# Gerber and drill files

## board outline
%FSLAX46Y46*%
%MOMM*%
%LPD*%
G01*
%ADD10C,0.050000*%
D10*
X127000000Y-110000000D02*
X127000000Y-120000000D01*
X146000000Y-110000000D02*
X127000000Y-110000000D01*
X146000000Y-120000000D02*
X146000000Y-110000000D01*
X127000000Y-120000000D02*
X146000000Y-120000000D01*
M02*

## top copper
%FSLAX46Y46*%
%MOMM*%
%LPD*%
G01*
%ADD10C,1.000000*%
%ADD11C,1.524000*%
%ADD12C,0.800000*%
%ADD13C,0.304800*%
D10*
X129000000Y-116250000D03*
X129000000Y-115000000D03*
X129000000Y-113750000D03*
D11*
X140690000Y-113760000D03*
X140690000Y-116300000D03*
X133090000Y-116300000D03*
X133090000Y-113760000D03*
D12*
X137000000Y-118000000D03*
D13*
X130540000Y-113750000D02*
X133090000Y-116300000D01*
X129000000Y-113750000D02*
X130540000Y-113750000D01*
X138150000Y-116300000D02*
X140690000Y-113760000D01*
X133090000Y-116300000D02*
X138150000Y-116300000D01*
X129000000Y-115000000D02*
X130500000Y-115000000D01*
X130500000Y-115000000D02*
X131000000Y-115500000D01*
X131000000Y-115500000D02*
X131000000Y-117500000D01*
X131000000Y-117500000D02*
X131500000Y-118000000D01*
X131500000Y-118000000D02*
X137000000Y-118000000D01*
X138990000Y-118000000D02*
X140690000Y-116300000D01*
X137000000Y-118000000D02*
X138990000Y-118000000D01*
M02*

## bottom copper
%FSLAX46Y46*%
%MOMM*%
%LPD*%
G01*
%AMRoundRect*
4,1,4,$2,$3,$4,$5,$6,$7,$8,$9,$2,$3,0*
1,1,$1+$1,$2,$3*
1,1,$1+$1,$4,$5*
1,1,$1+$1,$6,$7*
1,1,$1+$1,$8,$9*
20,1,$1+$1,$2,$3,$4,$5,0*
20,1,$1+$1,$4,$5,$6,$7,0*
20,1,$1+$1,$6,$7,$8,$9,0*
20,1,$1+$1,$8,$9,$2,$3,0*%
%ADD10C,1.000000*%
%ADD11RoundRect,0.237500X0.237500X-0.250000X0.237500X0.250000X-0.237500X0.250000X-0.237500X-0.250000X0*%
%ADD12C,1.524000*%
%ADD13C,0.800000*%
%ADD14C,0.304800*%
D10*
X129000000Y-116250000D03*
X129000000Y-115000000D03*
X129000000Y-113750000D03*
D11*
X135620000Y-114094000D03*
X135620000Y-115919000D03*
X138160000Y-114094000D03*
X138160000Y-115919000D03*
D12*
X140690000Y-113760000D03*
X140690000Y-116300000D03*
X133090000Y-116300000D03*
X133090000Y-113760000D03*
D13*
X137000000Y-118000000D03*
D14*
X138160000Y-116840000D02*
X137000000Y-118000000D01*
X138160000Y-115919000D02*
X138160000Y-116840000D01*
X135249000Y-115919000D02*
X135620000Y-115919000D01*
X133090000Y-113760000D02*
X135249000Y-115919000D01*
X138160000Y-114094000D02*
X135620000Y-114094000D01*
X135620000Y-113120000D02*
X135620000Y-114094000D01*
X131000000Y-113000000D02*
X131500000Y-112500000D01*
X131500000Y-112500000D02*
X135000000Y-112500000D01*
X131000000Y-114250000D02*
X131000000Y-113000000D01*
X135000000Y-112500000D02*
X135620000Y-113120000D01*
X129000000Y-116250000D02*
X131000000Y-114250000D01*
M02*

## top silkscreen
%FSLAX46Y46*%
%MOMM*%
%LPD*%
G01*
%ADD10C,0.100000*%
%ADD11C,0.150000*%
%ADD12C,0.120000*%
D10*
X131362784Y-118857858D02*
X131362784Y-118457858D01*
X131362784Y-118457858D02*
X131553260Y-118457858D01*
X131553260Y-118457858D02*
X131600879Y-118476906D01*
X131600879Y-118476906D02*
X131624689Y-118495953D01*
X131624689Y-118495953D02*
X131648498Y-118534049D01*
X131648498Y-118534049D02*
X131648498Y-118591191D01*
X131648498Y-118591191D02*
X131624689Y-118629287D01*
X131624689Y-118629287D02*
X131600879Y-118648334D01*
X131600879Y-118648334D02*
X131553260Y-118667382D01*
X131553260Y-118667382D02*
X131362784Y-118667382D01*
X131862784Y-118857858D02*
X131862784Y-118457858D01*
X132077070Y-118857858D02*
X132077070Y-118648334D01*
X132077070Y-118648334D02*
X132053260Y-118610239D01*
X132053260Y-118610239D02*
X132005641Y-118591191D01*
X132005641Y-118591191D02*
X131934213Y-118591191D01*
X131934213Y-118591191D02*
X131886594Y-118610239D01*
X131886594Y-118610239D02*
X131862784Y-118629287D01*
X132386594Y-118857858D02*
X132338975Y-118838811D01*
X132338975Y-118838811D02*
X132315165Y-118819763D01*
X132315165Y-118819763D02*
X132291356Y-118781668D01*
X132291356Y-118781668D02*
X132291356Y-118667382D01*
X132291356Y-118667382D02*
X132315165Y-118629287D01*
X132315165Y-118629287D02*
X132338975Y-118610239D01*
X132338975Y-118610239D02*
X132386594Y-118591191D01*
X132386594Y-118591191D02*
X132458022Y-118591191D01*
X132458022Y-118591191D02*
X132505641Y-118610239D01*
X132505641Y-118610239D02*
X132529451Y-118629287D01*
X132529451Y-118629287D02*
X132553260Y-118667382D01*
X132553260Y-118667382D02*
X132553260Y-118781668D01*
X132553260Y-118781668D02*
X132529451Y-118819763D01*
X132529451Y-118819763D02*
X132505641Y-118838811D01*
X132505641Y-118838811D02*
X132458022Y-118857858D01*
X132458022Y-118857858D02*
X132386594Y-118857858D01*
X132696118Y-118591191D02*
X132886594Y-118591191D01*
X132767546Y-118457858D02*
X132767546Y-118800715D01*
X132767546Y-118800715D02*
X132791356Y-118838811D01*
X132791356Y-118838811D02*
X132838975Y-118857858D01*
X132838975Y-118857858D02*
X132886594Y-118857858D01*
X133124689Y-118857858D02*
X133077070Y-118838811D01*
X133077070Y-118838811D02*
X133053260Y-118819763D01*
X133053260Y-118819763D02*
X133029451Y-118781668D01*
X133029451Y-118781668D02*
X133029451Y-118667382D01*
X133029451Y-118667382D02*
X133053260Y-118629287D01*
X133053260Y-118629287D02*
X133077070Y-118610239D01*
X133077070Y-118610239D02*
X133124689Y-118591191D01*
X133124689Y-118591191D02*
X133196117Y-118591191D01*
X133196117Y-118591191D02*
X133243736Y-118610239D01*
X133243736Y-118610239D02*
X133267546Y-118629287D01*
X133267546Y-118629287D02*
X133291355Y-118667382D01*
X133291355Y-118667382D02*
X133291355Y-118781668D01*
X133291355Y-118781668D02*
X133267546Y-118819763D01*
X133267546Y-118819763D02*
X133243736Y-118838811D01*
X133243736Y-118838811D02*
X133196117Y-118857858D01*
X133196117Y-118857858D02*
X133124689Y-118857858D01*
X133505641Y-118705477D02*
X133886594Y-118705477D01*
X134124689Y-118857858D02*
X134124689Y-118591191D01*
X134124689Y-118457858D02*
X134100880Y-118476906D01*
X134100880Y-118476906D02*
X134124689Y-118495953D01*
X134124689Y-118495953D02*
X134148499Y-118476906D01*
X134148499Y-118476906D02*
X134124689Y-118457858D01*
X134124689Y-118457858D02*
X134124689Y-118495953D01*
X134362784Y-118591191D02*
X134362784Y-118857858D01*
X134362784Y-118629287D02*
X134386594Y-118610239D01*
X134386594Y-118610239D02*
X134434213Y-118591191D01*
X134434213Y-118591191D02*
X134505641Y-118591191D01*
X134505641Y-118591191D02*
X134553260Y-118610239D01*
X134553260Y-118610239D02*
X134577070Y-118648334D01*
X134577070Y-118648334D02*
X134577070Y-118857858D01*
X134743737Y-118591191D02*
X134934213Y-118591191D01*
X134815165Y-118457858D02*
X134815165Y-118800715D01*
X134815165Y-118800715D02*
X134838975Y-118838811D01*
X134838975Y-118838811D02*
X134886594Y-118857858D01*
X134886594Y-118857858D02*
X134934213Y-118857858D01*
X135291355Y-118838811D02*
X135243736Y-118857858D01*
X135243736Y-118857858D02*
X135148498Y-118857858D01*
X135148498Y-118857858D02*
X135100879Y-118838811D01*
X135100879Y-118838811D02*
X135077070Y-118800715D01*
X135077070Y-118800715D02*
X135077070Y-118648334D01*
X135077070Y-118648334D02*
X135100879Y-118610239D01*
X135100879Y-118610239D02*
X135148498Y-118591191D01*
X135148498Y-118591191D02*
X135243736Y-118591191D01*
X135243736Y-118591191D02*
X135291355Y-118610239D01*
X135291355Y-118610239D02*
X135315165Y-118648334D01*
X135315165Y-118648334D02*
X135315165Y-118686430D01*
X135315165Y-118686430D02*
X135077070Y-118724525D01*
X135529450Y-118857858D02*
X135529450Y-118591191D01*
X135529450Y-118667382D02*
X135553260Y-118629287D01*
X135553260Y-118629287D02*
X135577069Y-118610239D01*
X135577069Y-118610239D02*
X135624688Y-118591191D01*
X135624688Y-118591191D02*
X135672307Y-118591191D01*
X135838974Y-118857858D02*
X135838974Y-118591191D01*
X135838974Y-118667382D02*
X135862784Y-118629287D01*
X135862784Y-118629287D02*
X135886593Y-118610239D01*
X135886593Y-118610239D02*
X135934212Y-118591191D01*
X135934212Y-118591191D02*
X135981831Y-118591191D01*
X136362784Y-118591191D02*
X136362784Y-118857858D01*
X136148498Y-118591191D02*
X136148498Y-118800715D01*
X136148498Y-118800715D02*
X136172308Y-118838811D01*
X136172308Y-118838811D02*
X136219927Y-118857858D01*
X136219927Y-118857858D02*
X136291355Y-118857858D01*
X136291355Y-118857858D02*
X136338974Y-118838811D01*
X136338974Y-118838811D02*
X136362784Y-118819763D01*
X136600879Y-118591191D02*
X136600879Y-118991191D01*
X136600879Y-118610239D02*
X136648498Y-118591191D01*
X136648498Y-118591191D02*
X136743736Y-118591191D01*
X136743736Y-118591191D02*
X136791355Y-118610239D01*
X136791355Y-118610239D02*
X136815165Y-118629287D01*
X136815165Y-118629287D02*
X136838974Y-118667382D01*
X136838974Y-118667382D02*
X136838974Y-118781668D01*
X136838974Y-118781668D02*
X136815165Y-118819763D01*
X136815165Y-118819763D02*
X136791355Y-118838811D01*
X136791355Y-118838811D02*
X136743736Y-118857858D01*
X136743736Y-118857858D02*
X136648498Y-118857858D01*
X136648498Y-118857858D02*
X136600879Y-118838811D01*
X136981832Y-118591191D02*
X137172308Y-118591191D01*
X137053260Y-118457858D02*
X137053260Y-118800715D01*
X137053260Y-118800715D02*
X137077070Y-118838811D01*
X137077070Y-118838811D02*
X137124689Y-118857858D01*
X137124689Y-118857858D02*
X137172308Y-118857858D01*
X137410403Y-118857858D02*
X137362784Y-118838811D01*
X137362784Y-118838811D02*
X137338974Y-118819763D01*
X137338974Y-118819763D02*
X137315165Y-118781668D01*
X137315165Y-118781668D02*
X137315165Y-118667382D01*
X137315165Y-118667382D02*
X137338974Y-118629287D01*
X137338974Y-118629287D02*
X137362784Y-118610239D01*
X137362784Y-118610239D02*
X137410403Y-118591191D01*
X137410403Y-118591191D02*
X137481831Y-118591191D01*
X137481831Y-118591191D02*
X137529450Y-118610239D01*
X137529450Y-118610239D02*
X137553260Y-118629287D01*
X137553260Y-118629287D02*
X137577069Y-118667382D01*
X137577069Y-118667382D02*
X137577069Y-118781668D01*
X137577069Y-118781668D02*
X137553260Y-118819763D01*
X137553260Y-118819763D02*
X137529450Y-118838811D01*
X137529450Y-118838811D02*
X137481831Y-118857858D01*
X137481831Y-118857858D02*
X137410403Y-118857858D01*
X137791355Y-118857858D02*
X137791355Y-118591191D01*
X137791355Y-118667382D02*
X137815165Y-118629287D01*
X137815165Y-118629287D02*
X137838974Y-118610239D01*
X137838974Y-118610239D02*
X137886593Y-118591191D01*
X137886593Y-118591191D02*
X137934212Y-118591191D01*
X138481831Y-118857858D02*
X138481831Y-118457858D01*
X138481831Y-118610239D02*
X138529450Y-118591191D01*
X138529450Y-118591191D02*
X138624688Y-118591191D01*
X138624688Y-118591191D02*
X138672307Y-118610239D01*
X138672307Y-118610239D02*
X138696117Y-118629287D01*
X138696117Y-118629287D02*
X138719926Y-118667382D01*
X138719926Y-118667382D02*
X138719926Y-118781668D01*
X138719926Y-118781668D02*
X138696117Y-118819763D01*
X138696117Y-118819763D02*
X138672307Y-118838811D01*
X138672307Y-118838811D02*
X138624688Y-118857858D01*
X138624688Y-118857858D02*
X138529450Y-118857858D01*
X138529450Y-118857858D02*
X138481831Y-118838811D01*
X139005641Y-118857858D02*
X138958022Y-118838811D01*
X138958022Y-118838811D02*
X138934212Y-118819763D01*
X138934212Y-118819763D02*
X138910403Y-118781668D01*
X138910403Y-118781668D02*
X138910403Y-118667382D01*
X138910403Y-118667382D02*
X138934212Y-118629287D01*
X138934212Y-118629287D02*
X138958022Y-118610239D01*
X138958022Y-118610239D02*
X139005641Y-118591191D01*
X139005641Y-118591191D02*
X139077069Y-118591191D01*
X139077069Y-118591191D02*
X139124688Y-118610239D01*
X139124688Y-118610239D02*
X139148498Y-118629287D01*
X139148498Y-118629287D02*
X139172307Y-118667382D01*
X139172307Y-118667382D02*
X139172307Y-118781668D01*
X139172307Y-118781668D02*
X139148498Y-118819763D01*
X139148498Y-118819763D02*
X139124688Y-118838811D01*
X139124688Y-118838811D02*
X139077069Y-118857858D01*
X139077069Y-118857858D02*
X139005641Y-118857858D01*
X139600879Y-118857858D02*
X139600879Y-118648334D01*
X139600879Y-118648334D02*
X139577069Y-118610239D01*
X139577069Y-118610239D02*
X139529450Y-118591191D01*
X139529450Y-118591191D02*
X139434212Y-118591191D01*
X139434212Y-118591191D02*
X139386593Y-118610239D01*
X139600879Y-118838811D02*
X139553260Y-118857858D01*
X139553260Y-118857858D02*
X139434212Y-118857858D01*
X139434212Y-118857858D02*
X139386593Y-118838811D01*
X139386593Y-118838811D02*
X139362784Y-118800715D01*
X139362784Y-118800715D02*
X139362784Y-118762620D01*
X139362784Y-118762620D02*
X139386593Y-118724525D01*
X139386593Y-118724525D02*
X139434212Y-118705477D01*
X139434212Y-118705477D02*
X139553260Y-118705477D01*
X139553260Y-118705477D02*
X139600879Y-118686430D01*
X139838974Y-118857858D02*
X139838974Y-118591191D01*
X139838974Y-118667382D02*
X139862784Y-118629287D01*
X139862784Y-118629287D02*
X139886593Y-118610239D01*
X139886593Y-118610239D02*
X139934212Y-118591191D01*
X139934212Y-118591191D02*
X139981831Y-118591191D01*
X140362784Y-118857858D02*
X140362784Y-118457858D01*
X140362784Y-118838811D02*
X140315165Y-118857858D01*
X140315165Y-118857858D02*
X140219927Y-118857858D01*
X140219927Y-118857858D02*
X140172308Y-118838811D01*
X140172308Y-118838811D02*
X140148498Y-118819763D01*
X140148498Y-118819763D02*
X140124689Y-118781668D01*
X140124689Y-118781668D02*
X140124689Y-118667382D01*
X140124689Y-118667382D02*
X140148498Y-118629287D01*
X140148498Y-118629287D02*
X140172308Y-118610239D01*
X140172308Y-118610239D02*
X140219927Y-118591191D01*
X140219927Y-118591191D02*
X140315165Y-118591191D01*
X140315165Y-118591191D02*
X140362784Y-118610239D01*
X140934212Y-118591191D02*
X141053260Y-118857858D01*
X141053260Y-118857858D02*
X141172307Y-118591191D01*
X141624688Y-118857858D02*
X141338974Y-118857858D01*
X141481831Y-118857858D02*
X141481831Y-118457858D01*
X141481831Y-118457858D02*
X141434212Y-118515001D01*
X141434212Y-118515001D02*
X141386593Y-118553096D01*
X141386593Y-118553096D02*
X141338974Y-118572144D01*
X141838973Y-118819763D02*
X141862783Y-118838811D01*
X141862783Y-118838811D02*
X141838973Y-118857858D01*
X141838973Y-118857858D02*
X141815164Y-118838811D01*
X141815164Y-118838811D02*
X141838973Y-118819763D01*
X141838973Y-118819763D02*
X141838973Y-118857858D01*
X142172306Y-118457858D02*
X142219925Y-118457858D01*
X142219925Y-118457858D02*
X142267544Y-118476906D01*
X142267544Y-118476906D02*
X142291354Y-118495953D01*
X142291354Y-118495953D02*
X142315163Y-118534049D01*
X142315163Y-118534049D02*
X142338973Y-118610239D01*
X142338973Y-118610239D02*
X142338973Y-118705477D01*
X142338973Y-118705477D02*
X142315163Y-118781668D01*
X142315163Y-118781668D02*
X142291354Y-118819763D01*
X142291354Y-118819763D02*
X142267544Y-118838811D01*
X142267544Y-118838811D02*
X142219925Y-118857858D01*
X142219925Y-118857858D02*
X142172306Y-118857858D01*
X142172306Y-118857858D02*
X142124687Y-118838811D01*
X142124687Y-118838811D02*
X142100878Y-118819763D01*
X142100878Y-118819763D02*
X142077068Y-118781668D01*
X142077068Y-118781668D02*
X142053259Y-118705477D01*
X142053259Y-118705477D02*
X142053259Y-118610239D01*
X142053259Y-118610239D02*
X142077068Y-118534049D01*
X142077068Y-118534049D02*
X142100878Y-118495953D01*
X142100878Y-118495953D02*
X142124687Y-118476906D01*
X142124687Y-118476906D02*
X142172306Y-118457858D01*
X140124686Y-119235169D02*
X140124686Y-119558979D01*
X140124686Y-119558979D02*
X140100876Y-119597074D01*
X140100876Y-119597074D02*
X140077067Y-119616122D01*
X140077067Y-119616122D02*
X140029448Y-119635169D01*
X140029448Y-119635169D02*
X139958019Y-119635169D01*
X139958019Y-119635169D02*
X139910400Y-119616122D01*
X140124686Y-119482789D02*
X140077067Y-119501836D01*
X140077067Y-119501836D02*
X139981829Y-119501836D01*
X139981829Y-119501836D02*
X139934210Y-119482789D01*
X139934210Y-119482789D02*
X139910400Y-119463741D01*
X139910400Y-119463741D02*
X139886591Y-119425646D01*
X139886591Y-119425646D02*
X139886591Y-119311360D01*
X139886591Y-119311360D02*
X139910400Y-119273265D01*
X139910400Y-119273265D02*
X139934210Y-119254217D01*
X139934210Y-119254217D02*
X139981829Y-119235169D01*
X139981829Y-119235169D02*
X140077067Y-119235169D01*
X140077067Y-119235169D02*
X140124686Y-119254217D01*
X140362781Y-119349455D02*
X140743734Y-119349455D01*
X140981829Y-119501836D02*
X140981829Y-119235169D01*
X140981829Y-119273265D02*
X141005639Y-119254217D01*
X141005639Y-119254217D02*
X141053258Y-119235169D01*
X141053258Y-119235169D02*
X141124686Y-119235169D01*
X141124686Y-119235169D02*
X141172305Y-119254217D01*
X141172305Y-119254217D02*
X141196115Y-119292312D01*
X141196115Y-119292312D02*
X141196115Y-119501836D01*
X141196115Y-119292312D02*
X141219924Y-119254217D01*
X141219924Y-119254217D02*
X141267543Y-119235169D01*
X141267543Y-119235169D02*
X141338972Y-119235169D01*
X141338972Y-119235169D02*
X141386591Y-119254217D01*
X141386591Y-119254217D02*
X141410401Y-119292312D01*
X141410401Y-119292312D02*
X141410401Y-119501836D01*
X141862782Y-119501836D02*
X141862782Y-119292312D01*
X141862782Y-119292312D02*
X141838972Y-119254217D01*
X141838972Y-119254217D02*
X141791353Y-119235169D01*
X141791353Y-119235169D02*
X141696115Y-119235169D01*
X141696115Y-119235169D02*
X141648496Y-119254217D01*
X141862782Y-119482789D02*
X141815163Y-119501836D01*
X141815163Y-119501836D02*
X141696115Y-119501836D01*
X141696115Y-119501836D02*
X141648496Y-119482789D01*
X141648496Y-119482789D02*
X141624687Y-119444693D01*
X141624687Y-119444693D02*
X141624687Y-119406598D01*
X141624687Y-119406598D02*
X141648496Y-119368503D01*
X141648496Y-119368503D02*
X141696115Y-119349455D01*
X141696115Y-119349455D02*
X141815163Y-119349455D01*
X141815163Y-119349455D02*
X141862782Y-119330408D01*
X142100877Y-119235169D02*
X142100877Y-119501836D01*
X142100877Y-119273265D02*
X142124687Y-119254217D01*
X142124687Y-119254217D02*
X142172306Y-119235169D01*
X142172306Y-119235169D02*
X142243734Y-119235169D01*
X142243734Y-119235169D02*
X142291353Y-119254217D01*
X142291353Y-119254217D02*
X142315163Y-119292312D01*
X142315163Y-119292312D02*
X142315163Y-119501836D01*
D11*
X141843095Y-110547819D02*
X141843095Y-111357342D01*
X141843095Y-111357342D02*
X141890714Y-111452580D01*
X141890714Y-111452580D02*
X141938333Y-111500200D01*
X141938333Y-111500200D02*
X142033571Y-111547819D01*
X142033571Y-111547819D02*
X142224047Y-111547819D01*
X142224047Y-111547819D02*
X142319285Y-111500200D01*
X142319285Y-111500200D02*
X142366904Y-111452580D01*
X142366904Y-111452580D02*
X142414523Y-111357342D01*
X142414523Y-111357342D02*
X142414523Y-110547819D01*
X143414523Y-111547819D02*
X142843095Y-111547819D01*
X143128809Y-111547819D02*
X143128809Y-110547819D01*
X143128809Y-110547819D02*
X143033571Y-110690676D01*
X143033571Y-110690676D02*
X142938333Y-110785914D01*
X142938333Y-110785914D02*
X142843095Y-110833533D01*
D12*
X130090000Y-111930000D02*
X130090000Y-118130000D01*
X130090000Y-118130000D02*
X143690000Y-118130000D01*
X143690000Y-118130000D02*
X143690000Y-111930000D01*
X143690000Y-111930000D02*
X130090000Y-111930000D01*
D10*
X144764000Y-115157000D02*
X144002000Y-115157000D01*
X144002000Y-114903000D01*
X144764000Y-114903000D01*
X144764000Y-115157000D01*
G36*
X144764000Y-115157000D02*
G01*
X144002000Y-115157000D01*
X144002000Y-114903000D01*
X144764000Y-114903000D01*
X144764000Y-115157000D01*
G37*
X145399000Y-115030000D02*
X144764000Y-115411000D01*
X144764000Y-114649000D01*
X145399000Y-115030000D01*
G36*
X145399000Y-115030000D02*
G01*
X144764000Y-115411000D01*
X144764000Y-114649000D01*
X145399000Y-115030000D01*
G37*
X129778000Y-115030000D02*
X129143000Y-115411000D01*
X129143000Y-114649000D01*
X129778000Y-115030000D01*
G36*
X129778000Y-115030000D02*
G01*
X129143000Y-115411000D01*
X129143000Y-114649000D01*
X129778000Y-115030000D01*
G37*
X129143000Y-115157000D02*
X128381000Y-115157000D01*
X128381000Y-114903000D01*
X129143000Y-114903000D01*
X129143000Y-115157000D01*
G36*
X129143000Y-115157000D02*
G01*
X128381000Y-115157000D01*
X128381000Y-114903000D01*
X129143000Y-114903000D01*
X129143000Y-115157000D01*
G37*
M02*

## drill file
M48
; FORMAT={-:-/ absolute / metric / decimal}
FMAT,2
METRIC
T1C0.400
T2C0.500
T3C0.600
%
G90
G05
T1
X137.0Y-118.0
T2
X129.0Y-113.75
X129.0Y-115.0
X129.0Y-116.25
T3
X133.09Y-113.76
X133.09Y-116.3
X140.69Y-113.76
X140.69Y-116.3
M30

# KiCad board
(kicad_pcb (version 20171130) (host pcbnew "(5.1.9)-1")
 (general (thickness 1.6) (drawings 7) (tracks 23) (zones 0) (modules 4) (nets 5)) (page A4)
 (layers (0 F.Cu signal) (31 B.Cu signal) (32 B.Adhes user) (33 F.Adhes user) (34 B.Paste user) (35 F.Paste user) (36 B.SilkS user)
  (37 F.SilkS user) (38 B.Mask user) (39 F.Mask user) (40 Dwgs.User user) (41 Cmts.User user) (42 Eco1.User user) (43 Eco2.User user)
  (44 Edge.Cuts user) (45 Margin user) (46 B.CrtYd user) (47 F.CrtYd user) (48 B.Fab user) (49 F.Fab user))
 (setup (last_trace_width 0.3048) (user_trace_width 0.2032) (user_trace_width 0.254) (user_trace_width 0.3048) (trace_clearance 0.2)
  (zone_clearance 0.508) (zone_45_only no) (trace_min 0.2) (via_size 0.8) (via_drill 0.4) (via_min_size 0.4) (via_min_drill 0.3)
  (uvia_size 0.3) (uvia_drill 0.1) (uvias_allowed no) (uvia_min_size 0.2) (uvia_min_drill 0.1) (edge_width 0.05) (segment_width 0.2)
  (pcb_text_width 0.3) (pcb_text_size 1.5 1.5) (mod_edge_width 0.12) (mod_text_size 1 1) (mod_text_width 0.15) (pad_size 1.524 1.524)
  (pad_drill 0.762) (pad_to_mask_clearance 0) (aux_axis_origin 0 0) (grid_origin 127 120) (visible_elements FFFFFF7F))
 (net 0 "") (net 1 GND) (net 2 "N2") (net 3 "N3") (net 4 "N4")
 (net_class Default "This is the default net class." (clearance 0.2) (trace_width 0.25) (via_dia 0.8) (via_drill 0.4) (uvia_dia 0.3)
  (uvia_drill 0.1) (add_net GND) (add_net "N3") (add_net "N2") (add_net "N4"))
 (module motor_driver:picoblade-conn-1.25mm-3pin (layer B.Cu) (at 129 115 270)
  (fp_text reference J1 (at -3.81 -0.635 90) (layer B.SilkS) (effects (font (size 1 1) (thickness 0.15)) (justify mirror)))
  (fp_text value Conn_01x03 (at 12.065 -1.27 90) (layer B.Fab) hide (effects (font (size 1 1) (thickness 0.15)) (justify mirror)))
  (pad 3 thru_hole circle (at 1.25 0 270) (size 1 1) (drill 0.5) (layers *.Cu *.Mask) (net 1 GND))
  (pad 2 thru_hole circle (at 0 0 270) (size 1 1) (drill 0.5) (layers *.Cu *.Mask) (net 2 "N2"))
  (pad 1 thru_hole circle (at -1.25 0 270) (size 1 1) (drill 0.5) (layers *.Cu *.Mask) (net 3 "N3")))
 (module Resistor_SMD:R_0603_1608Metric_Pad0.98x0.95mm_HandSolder (layer B.Cu) (at 135.62 115.0065 90)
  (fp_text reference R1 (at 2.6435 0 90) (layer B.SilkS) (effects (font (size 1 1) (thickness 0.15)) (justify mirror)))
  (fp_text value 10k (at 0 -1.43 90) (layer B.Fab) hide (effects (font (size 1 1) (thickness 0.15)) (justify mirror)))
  (pad 2 smd roundrect (at 0.9125 0 90) (size 0.975 0.95) (layers B.Cu B.Paste B.Mask) (roundrect_rratio 0.25) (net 1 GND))
  (pad 1 smd roundrect (at -0.9125 0 90) (size 0.975 0.95) (layers B.Cu B.Paste B.Mask) (roundrect_rratio 0.25) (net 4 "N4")))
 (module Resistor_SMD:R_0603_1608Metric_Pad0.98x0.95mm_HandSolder (layer B.Cu) (at 138.16 115.0065 90)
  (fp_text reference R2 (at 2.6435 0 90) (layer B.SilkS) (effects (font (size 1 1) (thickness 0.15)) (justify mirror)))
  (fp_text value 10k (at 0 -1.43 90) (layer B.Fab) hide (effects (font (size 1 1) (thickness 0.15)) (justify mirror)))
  (pad 2 smd roundrect (at 0.9125 0 90) (size 0.975 0.95) (layers B.Cu B.Paste B.Mask) (roundrect_rratio 0.25) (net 1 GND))
  (pad 1 smd roundrect (at -0.9125 0 90) (size 0.975 0.95) (layers B.Cu B.Paste B.Mask) (roundrect_rratio 0.25) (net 2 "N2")))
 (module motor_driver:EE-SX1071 (layer F.Cu) (at 136.89 115.03)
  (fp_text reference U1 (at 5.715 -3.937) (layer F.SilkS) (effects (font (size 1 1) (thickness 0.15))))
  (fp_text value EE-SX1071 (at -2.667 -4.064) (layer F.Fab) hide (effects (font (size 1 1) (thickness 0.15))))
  (fp_line (start -6.8 -3.1) (end -6.8 3.1) (layer F.SilkS) (width 0.12))
  (fp_line (start -6.8 3.1) (end 6.8 3.1) (layer F.SilkS) (width 0.12))
  (fp_line (start 6.8 3.1) (end 6.8 -3.1) (layer F.SilkS) (width 0.12))
  (fp_line (start 6.8 -3.1) (end -6.8 -3.1) (layer F.SilkS) (width 0.12))
  (fp_poly (pts (xy 7.874 0.127) (xy 7.112 0.127) (xy 7.112 -0.127) (xy 7.874 -0.127)) (layer F.SilkS) (width 0.1))
  (fp_poly (pts (xy 8.509 0) (xy 7.874 0.381) (xy 7.874 -0.381)) (layer F.SilkS) (width 0.1))
  (fp_poly (pts (xy -7.112 0) (xy -7.747 0.381) (xy -7.747 -0.381)) (layer F.SilkS) (width 0.1))
  (fp_poly (pts (xy -7.747 0.127) (xy -8.509 0.127) (xy -8.509 -0.127) (xy -7.747 -0.127)) (layer F.SilkS) (width 0.1))
  (pad 4 thru_hole circle (at 3.8 -1.27) (size 1.524 1.524) (drill 0.6) (layers *.Cu *.Mask) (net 3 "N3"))
  (pad 3 thru_hole circle (at 3.8 1.27) (size 1.524 1.524) (drill 0.6) (layers *.Cu *.Mask) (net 2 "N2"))
  (pad 2 thru_hole circle (at -3.8 1.27) (size 1.524 1.524) (drill 0.6) (layers *.Cu *.Mask) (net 3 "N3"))
  (pad 1 thru_hole circle (at -3.8 -1.27) (size 1.524 1.524) (drill 0.6) (layers *.Cu *.Mask) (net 4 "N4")))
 (gr_line (start 127 110) (end 127 120) (layer Edge.Cuts) (width 0.05))
 (gr_line (start 146 110) (end 127 110) (layer Edge.Cuts) (width 0.05))
 (gr_line (start 146 120) (end 146 110) (layer Edge.Cuts) (width 0.05))
 (gr_line (start 127 120) (end 146 120) (layer Edge.Cuts) (width 0.05))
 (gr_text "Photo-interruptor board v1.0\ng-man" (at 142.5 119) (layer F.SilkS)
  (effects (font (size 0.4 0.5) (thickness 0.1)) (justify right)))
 (segment (start 130.54 113.75) (end 133.09 116.3) (width 0.3048) (layer F.Cu) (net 3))
 (segment (start 129 113.75) (end 130.54 113.75) (width 0.3048) (layer F.Cu) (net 3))
 (segment (start 138.15 116.3) (end 140.69 113.76) (width 0.3048) (layer F.Cu) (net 3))
 (segment (start 133.09 116.3) (end 138.15 116.3) (width 0.3048) (layer F.Cu) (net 3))
 (via (at 137 118) (size 0.8) (drill 0.4) (layers F.Cu B.Cu) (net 2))
 (segment (start 129 115) (end 130.5 115) (width 0.3048) (layer F.Cu) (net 2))
 (segment (start 130.5 115) (end 131 115.5) (width 0.3048) (layer F.Cu) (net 2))
 (segment (start 131 115.5) (end 131 117.5) (width 0.3048) (layer F.Cu) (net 2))
 (segment (start 131 117.5) (end 131.5 118) (width 0.3048) (layer F.Cu) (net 2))
 (segment (start 131.5 118) (end 137 118) (width 0.3048) (layer F.Cu) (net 2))
 (segment (start 138.99 118) (end 140.69 116.3) (width 0.3048) (layer F.Cu) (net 2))
 (segment (start 137 118) (end 138.99 118) (width 0.3048) (layer F.Cu) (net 2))
 (segment (start 138.16 116.84) (end 137 118) (width 0.3048) (layer B.Cu) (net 2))
 (segment (start 138.16 115.919) (end 138.16 116.84) (width 0.3048) (layer B.Cu) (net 2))
 (segment (start 135.249 115.919) (end 135.62 115.919) (width 0.3048) (layer B.Cu) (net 4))
 (segment (start 133.09 113.76) (end 135.249 115.919) (width 0.3048) (layer B.Cu) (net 4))
 (segment (start 138.16 114.094) (end 135.62 114.094) (width 0.3048) (layer B.Cu) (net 1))
 (segment (start 135.62 113.12) (end 135.62 114.094) (width 0.3048) (layer B.Cu) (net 1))
 (segment (start 131 113) (end 131.5 112.5) (width 0.3048) (layer B.Cu) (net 1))
 (segment (start 131.5 112.5) (end 135 112.5) (width 0.3048) (layer B.Cu) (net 1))
 (segment (start 131 114.25) (end 131 113) (width 0.3048) (layer B.Cu) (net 1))
 (segment (start 135 112.5) (end 135.62 113.12) (width 0.3048) (layer B.Cu) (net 1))
 (segment (start 129 116.25) (end 131 114.25) (width 0.3048) (layer B.Cu) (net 1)))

